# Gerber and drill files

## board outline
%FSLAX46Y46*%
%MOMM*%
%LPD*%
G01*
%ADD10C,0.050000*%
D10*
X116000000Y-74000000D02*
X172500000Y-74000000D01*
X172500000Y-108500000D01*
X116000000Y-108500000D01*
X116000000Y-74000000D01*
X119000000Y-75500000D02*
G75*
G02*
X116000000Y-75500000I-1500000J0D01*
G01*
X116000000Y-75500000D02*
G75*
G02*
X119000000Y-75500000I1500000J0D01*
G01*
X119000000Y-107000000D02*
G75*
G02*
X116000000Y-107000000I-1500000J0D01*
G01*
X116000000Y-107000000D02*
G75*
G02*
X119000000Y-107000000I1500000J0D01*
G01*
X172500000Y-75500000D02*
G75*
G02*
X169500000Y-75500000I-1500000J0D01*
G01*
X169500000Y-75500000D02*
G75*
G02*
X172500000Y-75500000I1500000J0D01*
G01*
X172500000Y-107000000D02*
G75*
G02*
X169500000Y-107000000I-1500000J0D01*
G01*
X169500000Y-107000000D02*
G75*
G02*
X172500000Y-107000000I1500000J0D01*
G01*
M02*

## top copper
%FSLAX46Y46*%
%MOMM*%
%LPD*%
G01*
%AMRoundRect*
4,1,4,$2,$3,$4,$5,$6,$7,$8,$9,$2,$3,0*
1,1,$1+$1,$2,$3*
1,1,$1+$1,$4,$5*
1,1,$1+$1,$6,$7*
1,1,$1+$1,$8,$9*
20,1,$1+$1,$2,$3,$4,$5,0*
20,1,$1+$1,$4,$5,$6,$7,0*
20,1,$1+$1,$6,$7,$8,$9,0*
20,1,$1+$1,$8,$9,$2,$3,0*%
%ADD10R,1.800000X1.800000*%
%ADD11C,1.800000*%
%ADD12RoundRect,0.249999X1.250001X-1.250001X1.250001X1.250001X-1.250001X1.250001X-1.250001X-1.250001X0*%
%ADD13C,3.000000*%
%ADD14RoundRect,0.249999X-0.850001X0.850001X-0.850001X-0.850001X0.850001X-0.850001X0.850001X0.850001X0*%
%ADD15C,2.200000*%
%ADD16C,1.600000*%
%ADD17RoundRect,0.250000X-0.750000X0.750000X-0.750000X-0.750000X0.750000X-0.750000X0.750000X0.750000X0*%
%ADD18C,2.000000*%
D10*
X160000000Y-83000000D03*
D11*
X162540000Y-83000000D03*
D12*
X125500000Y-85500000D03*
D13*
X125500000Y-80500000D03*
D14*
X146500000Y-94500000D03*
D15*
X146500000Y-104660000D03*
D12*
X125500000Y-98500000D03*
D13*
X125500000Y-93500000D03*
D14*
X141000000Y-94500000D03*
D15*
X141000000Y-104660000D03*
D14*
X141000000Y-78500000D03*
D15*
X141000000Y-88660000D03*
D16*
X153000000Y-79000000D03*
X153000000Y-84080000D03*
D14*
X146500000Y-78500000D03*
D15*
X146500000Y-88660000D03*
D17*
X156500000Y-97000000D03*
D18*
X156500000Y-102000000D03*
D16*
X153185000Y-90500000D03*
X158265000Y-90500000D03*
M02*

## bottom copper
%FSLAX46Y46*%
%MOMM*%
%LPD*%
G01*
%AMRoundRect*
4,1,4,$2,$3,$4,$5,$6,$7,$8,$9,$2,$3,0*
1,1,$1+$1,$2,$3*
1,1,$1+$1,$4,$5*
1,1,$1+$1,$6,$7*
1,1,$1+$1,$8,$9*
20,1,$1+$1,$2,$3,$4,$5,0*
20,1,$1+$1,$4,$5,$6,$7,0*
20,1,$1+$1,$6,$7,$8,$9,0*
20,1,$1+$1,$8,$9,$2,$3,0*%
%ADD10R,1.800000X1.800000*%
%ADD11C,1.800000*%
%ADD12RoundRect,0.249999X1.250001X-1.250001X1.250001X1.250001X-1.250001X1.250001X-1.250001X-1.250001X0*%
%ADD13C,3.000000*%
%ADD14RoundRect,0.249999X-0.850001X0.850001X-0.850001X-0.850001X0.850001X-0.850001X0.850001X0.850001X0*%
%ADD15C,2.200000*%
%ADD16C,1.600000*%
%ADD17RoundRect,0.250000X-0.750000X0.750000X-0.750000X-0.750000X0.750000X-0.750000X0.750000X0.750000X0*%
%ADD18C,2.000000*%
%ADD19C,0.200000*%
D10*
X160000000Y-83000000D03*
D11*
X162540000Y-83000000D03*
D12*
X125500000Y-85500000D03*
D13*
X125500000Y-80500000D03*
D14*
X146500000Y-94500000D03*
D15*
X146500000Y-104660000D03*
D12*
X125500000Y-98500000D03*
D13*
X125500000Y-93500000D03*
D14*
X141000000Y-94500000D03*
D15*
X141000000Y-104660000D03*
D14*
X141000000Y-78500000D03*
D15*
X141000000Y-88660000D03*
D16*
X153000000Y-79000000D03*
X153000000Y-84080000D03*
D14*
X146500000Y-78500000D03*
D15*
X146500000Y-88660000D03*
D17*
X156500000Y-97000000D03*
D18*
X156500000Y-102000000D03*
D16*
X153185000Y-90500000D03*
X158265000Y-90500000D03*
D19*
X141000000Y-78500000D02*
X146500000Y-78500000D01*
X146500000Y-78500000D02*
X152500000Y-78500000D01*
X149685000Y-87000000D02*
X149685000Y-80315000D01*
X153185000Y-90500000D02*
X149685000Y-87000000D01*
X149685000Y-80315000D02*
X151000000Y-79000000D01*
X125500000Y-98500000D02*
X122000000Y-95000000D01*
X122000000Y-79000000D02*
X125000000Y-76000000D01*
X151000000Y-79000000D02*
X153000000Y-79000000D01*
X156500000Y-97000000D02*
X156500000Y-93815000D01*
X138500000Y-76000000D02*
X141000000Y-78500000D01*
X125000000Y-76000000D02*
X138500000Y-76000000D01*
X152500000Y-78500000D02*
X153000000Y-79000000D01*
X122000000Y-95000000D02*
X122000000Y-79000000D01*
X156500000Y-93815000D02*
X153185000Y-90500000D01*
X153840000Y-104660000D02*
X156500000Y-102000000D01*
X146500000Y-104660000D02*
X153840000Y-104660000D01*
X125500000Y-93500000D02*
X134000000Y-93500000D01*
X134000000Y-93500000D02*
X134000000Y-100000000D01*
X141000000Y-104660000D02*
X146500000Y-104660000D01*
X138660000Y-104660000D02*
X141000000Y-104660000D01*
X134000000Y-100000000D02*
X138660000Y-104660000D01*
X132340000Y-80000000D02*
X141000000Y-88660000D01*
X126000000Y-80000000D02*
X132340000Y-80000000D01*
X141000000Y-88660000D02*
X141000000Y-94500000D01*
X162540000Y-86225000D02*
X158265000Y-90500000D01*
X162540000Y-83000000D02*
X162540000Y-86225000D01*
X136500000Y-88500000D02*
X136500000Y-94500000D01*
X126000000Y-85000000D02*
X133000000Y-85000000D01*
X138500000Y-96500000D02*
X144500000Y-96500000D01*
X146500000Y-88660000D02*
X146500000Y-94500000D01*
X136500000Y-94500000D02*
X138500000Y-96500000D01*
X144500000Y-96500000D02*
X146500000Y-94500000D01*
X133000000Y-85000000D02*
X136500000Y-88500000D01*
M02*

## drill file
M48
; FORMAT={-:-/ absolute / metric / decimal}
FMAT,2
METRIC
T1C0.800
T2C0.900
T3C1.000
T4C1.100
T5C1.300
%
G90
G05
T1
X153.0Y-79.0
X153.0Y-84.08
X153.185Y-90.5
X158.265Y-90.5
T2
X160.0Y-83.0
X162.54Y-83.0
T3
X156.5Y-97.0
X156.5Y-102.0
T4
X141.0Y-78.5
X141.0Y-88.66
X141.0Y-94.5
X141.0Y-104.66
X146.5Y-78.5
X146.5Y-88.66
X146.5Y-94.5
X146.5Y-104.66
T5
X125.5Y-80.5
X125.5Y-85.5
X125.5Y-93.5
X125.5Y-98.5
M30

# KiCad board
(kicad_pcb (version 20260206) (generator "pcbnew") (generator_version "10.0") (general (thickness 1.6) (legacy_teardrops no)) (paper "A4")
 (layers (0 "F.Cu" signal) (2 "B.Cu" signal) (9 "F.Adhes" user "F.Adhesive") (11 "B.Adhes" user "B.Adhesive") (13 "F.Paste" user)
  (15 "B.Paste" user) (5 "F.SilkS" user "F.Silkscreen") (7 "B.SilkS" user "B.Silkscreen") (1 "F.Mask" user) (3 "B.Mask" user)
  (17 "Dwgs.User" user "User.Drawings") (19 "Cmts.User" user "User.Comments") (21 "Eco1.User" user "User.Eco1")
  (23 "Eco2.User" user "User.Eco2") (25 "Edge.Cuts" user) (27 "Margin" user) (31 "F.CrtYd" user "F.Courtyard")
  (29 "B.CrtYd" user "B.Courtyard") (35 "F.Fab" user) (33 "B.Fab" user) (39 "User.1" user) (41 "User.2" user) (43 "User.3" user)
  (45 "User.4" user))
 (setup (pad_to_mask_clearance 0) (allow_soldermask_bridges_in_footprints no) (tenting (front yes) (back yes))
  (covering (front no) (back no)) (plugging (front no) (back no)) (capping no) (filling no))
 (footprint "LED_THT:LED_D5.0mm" (layer "F.Cu") (at 160 83)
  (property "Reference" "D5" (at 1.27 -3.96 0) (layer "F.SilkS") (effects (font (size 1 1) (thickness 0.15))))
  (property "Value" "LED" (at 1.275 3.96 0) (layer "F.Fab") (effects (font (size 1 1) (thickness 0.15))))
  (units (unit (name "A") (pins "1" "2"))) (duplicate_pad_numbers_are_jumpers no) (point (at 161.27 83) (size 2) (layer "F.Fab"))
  (pad "1" thru_hole rect (at 0 0) (size 1.8 1.8) (drill 0.9) (layers "*.Cu" "*.Mask") (remove_unused_layers no) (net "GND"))
  (pad "2" thru_hole circle (at 2.54 0) (size 1.8 1.8) (drill 0.9) (layers "*.Cu" "*.Mask") (remove_unused_layers no) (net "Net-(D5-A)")))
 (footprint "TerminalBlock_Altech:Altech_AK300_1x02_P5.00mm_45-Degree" (layer "F.Cu") (at 125.5 85.5 90)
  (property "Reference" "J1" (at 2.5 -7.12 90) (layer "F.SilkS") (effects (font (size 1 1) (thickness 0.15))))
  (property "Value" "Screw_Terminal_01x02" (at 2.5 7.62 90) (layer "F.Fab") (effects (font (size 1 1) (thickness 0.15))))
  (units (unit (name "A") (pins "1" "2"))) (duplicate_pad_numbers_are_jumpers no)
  (pad "1" thru_hole roundrect (at 0 0 90) (size 3 3) (drill 1.3) (layers "*.Cu" "*.Mask") (remove_unused_layers no)
   (roundrect_rratio 0.083333) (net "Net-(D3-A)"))
  (pad "2" thru_hole circle (at 5 0 90) (size 3 3) (drill 1.3) (layers "*.Cu" "*.Mask") (remove_unused_layers no) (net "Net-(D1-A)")))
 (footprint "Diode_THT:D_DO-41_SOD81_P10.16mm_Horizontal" (layer "F.Cu") (at 146.5 94.5 -90)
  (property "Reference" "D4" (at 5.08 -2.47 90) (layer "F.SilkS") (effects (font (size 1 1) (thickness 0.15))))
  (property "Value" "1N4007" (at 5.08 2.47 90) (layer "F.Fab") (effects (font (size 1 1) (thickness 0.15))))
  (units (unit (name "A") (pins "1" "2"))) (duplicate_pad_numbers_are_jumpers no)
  (pad "1" thru_hole roundrect (at 0 0 270) (size 2.2 2.2) (drill 1.1) (layers "*.Cu" "*.Mask") (remove_unused_layers no)
   (roundrect_rratio 0.113636) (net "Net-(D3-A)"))
  (pad "2" thru_hole circle (at 10.16 0 270) (size 2.2 2.2) (drill 1.1) (layers "*.Cu" "*.Mask") (remove_unused_layers no) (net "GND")))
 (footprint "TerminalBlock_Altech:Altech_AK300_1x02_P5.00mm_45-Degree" (layer "F.Cu") (at 125.5 98.5 90)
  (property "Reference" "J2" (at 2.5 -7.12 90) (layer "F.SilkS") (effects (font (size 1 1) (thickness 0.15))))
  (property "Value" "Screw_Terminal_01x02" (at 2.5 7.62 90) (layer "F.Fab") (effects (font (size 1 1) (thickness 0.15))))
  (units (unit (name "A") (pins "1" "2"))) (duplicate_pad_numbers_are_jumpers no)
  (pad "1" thru_hole roundrect (at 0 0 90) (size 3 3) (drill 1.3) (layers "*.Cu" "*.Mask") (remove_unused_layers no)
   (roundrect_rratio 0.083333) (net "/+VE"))
  (pad "2" thru_hole circle (at 5 0 90) (size 3 3) (drill 1.3) (layers "*.Cu" "*.Mask") (remove_unused_layers no) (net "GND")))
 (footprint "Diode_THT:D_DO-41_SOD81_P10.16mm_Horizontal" (layer "F.Cu") (at 141 94.5 -90)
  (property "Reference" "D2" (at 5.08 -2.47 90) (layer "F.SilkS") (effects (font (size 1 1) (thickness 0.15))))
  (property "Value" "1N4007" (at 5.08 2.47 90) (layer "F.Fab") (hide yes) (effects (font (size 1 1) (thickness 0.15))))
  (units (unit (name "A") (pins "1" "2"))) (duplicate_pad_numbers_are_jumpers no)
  (pad "1" thru_hole roundrect (at 0 0 270) (size 2.2 2.2) (drill 1.1) (layers "*.Cu" "*.Mask") (remove_unused_layers no)
   (roundrect_rratio 0.113636) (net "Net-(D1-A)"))
  (pad "2" thru_hole circle (at 10.16 0 270) (size 2.2 2.2) (drill 1.1) (layers "*.Cu" "*.Mask") (remove_unused_layers no) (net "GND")))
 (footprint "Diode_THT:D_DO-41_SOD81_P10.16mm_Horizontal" (layer "F.Cu") (at 141 78.5 -90)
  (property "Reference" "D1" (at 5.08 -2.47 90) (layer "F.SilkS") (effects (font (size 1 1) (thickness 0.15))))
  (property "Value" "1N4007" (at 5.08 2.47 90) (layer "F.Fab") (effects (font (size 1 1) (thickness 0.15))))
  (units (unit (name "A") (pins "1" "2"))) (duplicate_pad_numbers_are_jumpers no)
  (pad "1" thru_hole roundrect (at 0 0 270) (size 2.2 2.2) (drill 1.1) (layers "*.Cu" "*.Mask") (remove_unused_layers no)
   (roundrect_rratio 0.113636) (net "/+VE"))
  (pad "2" thru_hole circle (at 10.16 0 270) (size 2.2 2.2) (drill 1.1) (layers "*.Cu" "*.Mask") (remove_unused_layers no)
   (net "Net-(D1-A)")))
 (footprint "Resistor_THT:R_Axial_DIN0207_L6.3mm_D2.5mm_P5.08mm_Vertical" (layer "F.Cu") (at 153 79 -90)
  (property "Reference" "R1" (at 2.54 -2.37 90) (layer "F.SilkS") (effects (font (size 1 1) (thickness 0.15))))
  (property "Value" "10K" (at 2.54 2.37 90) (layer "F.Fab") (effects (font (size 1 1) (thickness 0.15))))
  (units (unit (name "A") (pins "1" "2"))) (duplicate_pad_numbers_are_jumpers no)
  (pad "1" thru_hole circle (at 0 0 270) (size 1.6 1.6) (drill 0.8) (layers "*.Cu" "*.Mask") (remove_unused_layers no) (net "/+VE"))
  (pad "2" thru_hole circle (at 5.08 0 270) (size 1.6 1.6) (drill 0.8) (layers "*.Cu" "*.Mask") (remove_unused_layers no) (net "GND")))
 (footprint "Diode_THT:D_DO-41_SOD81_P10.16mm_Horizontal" (layer "F.Cu") (at 146.5 78.5 -90)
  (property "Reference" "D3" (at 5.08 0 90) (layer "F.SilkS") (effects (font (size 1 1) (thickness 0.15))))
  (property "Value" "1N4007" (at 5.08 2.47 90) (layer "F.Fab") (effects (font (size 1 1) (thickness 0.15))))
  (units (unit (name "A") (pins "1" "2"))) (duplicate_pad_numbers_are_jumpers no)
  (pad "1" thru_hole roundrect (at 0 0 270) (size 2.2 2.2) (drill 1.1) (layers "*.Cu" "*.Mask") (remove_unused_layers no)
   (roundrect_rratio 0.113636) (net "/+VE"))
  (pad "2" thru_hole circle (at 10.16 0 270) (size 2.2 2.2) (drill 1.1) (layers "*.Cu" "*.Mask") (remove_unused_layers no)
   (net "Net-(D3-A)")))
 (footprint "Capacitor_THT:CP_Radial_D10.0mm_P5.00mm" (layer "F.Cu") (at 156.5 97 -90)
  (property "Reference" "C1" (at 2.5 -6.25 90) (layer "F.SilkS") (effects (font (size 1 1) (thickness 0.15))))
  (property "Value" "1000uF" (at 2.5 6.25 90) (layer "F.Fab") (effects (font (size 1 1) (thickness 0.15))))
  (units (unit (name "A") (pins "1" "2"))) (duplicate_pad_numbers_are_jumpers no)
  (pad "1" thru_hole roundrect (at 0 0 270) (size 2 2) (drill 1) (layers "*.Cu" "*.Mask") (remove_unused_layers no) (roundrect_rratio 0.125)
   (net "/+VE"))
  (pad "2" thru_hole circle (at 5 0 270) (size 2 2) (drill 1) (layers "*.Cu" "*.Mask") (remove_unused_layers no) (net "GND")))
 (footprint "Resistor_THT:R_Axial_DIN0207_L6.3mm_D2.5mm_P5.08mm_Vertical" (layer "F.Cu") (at 153.185 90.5)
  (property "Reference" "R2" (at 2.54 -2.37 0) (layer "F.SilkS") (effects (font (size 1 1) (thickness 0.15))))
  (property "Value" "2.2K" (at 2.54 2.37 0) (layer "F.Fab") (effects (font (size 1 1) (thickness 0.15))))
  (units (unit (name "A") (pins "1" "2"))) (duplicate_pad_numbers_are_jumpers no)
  (pad "1" thru_hole circle (at 0 0) (size 1.6 1.6) (drill 0.8) (layers "*.Cu" "*.Mask") (remove_unused_layers no) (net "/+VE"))
  (pad "2" thru_hole circle (at 5.08 0) (size 1.6 1.6) (drill 0.8) (layers "*.Cu" "*.Mask") (remove_unused_layers no) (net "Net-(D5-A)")))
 (gr_rect (start 116 74) (end 172.5 108.5) (stroke (width 0.05) (type default)) (fill no) (layer "Edge.Cuts"))
 (gr_circle (center 117.5 75.5) (end 119 75.5) (stroke (width 0.05) (type default)) (fill no) (layer "Edge.Cuts"))
 (gr_circle (center 117.5 107) (end 119 107) (stroke (width 0.05) (type default)) (fill no) (layer "Edge.Cuts"))
 (gr_circle (center 171 75.5) (end 172.5 75.5) (stroke (width 0.05) (type default)) (fill no) (layer "Edge.Cuts"))
 (gr_circle (center 171 107) (end 172.5 107) (stroke (width 0.05) (type default)) (fill no) (layer "Edge.Cuts"))
 (segment (start 141 78.5) (end 146.5 78.5) (width 0.2) (layer "B.Cu") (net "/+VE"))
 (segment (start 146.5 78.5) (end 152.5 78.5) (width 0.2) (layer "B.Cu") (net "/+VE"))
 (segment (start 149.685 87) (end 149.685 80.315) (width 0.2) (layer "B.Cu") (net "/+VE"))
 (segment (start 153.185 90.5) (end 149.685 87) (width 0.2) (layer "B.Cu") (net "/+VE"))
 (segment (start 149.685 80.315) (end 151 79) (width 0.2) (layer "B.Cu") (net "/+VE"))
 (segment (start 125.5 98.5) (end 122 95) (width 0.2) (layer "B.Cu") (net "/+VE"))
 (segment (start 122 79) (end 125 76) (width 0.2) (layer "B.Cu") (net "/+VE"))
 (segment (start 151 79) (end 153 79) (width 0.2) (layer "B.Cu") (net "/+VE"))
 (segment (start 156.5 97) (end 156.5 93.815) (width 0.2) (layer "B.Cu") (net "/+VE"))
 (segment (start 138.5 76) (end 141 78.5) (width 0.2) (layer "B.Cu") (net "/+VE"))
 (segment (start 125 76) (end 138.5 76) (width 0.2) (layer "B.Cu") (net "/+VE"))
 (segment (start 152.5 78.5) (end 153 79) (width 0.2) (layer "B.Cu") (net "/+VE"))
 (segment (start 122 95) (end 122 79) (width 0.2) (layer "B.Cu") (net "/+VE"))
 (segment (start 156.5 93.815) (end 153.185 90.5) (width 0.2) (layer "B.Cu") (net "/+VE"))
 (segment (start 153.84 104.66) (end 156.5 102) (width 0.2) (layer "B.Cu") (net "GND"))
 (segment (start 146.5 104.66) (end 153.84 104.66) (width 0.2) (layer "B.Cu") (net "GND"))
 (segment (start 125.5 93.5) (end 134 93.5) (width 0.2) (layer "B.Cu") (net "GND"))
 (segment (start 134 93.5) (end 134 100) (width 0.2) (layer "B.Cu") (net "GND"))
 (segment (start 141 104.66) (end 146.5 104.66) (width 0.2) (layer "B.Cu") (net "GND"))
 (segment (start 138.66 104.66) (end 141 104.66) (width 0.2) (layer "B.Cu") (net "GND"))
 (segment (start 134 100) (end 138.66 104.66) (width 0.2) (layer "B.Cu") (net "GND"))
 (segment (start 132.34 80) (end 141 88.66) (width 0.2) (layer "B.Cu") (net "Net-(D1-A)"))
 (segment (start 126 80) (end 132.34 80) (width 0.2) (layer "B.Cu") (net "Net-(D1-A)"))
 (segment (start 141 88.66) (end 141 94.5) (width 0.2) (layer "B.Cu") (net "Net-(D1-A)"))
 (segment (start 162.54 86.225) (end 158.265 90.5) (width 0.2) (layer "B.Cu") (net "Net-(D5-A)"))
 (segment (start 162.54 83) (end 162.54 86.225) (width 0.2) (layer "B.Cu") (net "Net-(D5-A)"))
 (segment (start 136.5 88.5) (end 136.5 94.5) (width 0.2) (layer "B.Cu") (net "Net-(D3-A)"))
 (segment (start 126 85) (end 133 85) (width 0.2) (layer "B.Cu") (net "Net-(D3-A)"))
 (segment (start 138.5 96.5) (end 144.5 96.5) (width 0.2) (layer "B.Cu") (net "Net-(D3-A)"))
 (segment (start 146.5 88.66) (end 146.5 94.5) (width 0.2) (layer "B.Cu") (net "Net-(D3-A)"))
 (segment (start 136.5 94.5) (end 138.5 96.5) (width 0.2) (layer "B.Cu") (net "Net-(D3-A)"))
 (segment (start 144.5 96.5) (end 146.5 94.5) (width 0.2) (layer "B.Cu") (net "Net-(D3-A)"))
 (segment (start 133 85) (end 136.5 88.5) (width 0.2) (layer "B.Cu") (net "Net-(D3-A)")))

